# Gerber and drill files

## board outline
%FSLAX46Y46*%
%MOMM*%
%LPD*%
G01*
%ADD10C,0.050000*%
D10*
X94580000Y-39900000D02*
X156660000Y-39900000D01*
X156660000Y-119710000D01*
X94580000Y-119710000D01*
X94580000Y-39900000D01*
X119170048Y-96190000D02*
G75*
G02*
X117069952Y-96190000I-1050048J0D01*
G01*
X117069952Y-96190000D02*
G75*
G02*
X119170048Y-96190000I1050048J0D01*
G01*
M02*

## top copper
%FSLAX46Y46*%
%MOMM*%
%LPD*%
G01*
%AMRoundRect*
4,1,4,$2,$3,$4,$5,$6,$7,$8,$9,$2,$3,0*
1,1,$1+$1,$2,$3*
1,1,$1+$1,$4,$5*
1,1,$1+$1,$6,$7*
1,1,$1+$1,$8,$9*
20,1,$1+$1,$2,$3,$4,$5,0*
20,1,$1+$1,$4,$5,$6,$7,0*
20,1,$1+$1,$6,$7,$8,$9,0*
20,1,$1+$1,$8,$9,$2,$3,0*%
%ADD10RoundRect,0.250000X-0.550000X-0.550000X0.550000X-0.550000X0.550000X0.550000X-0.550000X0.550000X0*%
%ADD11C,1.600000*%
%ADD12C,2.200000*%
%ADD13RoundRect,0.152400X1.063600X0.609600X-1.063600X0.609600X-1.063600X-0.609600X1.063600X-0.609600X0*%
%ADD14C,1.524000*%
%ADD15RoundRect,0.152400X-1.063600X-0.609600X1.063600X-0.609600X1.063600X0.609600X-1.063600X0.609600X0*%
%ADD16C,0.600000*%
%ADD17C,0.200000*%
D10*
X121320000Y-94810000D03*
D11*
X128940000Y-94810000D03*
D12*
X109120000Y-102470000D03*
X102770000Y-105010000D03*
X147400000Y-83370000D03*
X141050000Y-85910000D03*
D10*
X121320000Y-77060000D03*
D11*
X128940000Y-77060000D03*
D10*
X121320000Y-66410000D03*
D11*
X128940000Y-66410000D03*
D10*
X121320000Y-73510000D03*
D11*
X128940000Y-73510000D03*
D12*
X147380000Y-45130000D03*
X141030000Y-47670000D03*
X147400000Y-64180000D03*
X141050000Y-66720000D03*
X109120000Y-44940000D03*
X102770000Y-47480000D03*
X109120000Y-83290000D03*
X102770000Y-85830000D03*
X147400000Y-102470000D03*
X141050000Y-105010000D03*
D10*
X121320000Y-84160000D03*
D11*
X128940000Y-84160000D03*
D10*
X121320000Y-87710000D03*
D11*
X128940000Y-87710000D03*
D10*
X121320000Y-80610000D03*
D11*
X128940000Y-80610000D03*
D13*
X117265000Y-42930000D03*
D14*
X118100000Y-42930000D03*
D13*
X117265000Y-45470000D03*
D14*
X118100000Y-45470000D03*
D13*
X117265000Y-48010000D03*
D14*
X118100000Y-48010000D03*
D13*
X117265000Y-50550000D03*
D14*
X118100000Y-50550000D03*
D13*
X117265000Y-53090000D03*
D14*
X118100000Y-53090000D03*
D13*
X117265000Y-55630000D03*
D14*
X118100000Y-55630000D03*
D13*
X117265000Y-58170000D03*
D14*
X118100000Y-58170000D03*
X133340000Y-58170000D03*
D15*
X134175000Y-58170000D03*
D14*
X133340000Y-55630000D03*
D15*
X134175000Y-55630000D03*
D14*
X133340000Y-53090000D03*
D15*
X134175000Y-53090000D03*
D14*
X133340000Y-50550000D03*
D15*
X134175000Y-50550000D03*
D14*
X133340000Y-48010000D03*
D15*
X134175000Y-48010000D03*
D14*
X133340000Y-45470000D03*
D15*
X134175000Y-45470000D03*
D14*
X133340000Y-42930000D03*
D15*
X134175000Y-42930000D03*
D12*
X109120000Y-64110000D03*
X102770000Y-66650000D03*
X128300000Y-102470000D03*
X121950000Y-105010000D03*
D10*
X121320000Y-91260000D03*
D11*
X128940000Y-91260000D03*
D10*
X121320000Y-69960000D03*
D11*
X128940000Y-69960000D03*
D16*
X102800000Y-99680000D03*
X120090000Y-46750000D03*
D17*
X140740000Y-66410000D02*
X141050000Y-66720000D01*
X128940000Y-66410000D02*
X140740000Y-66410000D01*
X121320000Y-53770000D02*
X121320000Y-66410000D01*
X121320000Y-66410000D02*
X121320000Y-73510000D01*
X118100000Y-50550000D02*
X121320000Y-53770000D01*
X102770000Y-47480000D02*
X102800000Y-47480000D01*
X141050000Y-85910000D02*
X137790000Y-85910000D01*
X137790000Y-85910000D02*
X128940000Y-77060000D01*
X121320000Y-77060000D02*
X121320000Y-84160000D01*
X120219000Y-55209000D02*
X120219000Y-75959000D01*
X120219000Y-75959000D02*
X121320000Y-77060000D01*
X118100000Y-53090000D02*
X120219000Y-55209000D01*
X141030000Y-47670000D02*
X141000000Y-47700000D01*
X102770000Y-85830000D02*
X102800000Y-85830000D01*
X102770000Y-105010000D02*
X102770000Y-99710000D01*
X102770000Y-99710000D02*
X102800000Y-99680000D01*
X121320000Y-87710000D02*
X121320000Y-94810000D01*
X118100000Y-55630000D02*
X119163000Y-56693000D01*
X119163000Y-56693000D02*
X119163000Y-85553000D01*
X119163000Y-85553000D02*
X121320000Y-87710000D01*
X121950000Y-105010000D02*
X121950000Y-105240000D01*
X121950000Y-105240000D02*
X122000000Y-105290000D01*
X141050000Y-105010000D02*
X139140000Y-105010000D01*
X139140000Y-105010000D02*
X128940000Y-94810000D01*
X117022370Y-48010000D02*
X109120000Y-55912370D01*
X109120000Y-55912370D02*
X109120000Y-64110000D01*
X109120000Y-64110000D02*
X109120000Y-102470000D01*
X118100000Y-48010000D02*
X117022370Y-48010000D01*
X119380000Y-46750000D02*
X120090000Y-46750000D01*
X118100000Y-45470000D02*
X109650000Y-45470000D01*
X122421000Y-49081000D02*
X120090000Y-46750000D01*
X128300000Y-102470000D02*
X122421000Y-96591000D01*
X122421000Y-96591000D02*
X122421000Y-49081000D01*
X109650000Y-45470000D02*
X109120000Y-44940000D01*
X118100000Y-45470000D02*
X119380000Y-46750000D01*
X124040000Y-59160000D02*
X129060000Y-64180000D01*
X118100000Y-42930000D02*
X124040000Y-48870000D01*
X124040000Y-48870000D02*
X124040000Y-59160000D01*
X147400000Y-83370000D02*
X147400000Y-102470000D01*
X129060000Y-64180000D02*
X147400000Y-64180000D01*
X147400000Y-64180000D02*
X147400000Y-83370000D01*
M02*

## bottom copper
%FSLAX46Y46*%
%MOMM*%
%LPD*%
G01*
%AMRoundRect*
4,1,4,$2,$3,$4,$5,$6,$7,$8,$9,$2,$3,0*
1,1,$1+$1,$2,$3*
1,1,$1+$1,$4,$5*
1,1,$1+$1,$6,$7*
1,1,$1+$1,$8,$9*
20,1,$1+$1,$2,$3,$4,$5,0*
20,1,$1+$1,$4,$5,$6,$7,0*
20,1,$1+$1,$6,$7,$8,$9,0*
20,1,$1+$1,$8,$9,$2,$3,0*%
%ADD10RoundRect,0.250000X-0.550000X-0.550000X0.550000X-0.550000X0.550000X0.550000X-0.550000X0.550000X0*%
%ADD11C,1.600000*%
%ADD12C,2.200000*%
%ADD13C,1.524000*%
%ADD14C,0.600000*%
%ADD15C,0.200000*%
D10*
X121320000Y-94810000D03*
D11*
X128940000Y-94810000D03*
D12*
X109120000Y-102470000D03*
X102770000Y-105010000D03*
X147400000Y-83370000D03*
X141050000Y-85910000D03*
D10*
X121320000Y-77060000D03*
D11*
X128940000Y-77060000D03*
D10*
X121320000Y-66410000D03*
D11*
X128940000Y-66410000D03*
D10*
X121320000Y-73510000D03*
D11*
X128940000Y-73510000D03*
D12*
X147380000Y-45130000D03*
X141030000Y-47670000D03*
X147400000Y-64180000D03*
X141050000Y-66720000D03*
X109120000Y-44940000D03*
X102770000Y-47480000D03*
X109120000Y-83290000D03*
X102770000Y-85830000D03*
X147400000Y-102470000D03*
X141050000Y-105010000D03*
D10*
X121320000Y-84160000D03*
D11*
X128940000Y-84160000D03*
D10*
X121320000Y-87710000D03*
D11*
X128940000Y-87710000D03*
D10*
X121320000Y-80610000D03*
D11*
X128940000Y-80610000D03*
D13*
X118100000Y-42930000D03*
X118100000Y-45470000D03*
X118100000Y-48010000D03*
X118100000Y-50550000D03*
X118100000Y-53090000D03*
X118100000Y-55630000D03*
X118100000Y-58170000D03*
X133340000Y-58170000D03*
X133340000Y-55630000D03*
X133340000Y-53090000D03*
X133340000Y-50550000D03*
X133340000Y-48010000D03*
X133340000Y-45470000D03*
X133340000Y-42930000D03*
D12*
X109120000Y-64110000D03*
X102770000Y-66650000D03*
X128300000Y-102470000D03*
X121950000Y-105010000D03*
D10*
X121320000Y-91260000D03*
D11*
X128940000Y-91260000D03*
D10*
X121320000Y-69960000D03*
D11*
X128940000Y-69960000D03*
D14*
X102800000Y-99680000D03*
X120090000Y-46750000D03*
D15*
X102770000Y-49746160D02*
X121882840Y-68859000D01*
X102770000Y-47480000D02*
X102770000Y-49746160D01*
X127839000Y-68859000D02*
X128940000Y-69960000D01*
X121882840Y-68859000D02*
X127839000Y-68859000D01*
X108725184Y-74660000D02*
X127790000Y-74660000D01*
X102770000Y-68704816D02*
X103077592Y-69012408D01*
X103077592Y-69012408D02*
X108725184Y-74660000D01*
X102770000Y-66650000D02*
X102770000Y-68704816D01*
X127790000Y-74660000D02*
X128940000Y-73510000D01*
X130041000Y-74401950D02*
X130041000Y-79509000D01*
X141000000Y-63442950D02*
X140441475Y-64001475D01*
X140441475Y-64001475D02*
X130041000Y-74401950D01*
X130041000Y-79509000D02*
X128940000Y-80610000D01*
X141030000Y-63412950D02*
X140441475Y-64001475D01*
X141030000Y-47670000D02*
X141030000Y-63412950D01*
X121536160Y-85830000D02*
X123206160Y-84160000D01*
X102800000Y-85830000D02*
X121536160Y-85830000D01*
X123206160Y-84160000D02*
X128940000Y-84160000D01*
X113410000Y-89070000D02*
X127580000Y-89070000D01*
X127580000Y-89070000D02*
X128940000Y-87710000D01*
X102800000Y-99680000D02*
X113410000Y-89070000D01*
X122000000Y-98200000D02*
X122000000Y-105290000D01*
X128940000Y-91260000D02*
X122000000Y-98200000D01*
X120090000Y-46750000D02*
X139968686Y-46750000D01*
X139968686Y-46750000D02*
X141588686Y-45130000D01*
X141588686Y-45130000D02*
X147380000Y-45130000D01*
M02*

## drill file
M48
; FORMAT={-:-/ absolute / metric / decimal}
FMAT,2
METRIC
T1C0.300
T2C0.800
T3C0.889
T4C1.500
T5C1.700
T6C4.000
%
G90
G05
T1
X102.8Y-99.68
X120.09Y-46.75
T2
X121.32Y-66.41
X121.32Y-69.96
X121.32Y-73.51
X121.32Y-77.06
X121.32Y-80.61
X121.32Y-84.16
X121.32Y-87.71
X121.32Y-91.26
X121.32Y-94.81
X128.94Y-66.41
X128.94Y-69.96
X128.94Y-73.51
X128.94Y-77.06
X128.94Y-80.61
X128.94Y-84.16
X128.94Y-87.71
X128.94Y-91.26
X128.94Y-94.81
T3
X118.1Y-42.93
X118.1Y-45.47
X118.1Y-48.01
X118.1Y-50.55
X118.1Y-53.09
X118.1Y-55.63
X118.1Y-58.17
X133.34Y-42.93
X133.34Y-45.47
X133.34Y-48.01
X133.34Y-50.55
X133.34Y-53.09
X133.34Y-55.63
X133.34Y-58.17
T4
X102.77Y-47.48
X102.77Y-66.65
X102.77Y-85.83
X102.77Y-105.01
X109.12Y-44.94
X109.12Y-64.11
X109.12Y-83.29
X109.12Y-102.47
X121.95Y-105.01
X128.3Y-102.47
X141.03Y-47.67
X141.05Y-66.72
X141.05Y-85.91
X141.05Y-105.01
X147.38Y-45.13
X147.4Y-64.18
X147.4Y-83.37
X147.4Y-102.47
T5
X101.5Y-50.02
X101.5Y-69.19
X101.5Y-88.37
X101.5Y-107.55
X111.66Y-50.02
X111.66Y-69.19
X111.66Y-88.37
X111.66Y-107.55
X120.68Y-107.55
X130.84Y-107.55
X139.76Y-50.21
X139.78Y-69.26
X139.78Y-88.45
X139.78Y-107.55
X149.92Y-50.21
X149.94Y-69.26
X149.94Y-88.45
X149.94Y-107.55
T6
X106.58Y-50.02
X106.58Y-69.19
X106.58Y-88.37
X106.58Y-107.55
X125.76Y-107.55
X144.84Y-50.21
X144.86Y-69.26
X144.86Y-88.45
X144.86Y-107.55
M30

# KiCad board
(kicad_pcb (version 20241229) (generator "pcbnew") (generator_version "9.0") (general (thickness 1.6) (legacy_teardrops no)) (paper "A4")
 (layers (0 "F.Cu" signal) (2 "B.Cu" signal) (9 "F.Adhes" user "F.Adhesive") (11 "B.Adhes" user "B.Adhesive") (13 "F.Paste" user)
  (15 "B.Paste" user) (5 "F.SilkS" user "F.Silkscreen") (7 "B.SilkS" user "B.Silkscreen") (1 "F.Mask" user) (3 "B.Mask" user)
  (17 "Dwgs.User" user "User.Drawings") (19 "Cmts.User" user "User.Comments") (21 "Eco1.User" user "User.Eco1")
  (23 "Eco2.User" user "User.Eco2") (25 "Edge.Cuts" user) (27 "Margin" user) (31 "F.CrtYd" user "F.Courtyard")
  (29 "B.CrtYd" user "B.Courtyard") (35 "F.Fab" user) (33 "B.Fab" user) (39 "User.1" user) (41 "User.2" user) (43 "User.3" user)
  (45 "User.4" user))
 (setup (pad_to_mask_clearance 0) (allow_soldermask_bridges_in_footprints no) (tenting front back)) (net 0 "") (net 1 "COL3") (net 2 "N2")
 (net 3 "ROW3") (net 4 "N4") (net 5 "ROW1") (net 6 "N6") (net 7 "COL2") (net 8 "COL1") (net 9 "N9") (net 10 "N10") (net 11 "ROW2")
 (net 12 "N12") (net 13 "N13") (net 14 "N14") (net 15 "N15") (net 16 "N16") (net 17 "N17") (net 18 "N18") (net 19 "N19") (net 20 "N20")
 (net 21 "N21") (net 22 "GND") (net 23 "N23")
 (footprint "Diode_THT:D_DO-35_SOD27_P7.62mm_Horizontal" (layer "F.Cu") (at 121.32 94.81)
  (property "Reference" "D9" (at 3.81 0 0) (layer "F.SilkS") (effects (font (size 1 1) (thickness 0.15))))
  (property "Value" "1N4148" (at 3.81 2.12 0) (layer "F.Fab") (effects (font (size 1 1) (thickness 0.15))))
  (pad "1" thru_hole roundrect (at 0 0) (size 1.6 1.6) (drill 0.8) (layers "*.Cu" "*.Mask") (remove_unused_layers no)
   (roundrect_rratio 0.15625) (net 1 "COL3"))
  (pad "2" thru_hole circle (at 7.62 0) (size 1.6 1.6) (drill 0.8) (layers "*.Cu" "*.Mask") (remove_unused_layers no) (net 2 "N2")))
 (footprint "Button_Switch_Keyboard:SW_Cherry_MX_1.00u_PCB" (layer "F.Cu") (at 109.12 102.47)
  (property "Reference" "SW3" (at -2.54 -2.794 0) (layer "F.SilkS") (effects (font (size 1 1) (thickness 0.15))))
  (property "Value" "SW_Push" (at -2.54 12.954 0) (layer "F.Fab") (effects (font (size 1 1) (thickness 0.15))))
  (pad "" np_thru_hole circle (at -7.62 5.08) (size 1.7 1.7) (drill 1.7) (layers "*.Cu" "*.Mask"))
  (pad "" np_thru_hole circle (at -2.54 5.08) (size 4 4) (drill 4) (layers "*.Cu" "*.Mask"))
  (pad "" np_thru_hole circle (at 2.54 5.08) (size 1.7 1.7) (drill 1.7) (layers "*.Cu" "*.Mask"))
  (pad "1" thru_hole circle (at 0 0) (size 2.2 2.2) (drill 1.5) (layers "*.Cu" "*.Mask") (remove_unused_layers no) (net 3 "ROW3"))
  (pad "2" thru_hole circle (at -6.35 2.54) (size 2.2 2.2) (drill 1.5) (layers "*.Cu" "*.Mask") (remove_unused_layers no) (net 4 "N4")))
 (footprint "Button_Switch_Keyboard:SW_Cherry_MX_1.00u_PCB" (layer "F.Cu") (at 147.4 83.37)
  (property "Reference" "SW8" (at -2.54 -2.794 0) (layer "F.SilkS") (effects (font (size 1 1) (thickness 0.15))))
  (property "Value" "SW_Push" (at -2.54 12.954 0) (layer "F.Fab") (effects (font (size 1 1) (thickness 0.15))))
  (pad "" np_thru_hole circle (at -7.62 5.08) (size 1.7 1.7) (drill 1.7) (layers "*.Cu" "*.Mask"))
  (pad "" np_thru_hole circle (at -2.54 5.08) (size 4 4) (drill 4) (layers "*.Cu" "*.Mask"))
  (pad "" np_thru_hole circle (at 2.54 5.08) (size 1.7 1.7) (drill 1.7) (layers "*.Cu" "*.Mask"))
  (pad "1" thru_hole circle (at 0 0) (size 2.2 2.2) (drill 1.5) (layers "*.Cu" "*.Mask") (remove_unused_layers no) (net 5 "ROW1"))
  (pad "2" thru_hole circle (at -6.35 2.54) (size 2.2 2.2) (drill 1.5) (layers "*.Cu" "*.Mask") (remove_unused_layers no) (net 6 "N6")))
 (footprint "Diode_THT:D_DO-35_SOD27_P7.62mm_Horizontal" (layer "F.Cu") (at 121.32 77.06)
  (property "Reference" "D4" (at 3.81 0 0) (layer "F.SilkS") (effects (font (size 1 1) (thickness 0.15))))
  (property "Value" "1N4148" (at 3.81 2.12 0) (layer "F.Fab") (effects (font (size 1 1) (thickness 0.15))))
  (pad "1" thru_hole roundrect (at 0 0) (size 1.6 1.6) (drill 0.8) (layers "*.Cu" "*.Mask") (remove_unused_layers no)
   (roundrect_rratio 0.15625) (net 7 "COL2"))
  (pad "2" thru_hole circle (at 7.62 0) (size 1.6 1.6) (drill 0.8) (layers "*.Cu" "*.Mask") (remove_unused_layers no) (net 6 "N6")))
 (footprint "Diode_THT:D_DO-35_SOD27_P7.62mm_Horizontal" (layer "F.Cu") (at 121.32 66.41)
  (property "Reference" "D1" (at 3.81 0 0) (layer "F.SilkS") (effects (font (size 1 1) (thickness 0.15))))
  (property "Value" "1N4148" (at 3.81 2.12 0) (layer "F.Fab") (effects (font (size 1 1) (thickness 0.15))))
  (pad "1" thru_hole roundrect (at 0 0) (size 1.6 1.6) (drill 0.8) (layers "*.Cu" "*.Mask") (remove_unused_layers no)
   (roundrect_rratio 0.15625) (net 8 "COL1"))
  (pad "2" thru_hole circle (at 7.62 0) (size 1.6 1.6) (drill 0.8) (layers "*.Cu" "*.Mask") (remove_unused_layers no) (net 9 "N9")))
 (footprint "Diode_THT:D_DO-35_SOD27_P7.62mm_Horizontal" (layer "F.Cu") (at 121.32 73.51)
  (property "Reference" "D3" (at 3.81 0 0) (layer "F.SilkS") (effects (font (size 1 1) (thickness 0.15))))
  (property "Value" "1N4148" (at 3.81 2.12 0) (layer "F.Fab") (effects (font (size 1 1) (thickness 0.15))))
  (pad "1" thru_hole roundrect (at 0 0) (size 1.6 1.6) (drill 0.8) (layers "*.Cu" "*.Mask") (remove_unused_layers no)
   (roundrect_rratio 0.15625) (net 8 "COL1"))
  (pad "2" thru_hole circle (at 7.62 0) (size 1.6 1.6) (drill 0.8) (layers "*.Cu" "*.Mask") (remove_unused_layers no) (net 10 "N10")))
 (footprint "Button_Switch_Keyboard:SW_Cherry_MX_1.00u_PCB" (layer "F.Cu") (at 147.38 45.13)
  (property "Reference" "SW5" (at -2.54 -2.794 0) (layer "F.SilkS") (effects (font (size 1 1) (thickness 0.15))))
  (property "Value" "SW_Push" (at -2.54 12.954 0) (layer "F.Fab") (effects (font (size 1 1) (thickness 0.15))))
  (pad "" np_thru_hole circle (at -7.62 5.08) (size 1.7 1.7) (drill 1.7) (layers "*.Cu" "*.Mask"))
  (pad "" np_thru_hole circle (at -2.54 5.08) (size 4 4) (drill 4) (layers "*.Cu" "*.Mask"))
  (pad "" np_thru_hole circle (at 2.54 5.08) (size 1.7 1.7) (drill 1.7) (layers "*.Cu" "*.Mask"))
  (pad "1" thru_hole circle (at 0 0) (size 2.2 2.2) (drill 1.5) (layers "*.Cu" "*.Mask") (remove_unused_layers no) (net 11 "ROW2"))
  (pad "2" thru_hole circle (at -6.35 2.54) (size 2.2 2.2) (drill 1.5) (layers "*.Cu" "*.Mask") (remove_unused_layers no) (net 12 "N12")))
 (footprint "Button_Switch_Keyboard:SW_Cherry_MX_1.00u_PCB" (layer "F.Cu") (at 147.4 64.18)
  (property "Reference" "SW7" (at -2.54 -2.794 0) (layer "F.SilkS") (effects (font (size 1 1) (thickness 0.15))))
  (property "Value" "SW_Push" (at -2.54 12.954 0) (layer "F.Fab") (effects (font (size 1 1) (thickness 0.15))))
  (pad "" np_thru_hole circle (at -7.62 5.08) (size 1.7 1.7) (drill 1.7) (layers "*.Cu" "*.Mask"))
  (pad "" np_thru_hole circle (at -2.54 5.08) (size 4 4) (drill 4) (layers "*.Cu" "*.Mask"))
  (pad "" np_thru_hole circle (at 2.54 5.08) (size 1.7 1.7) (drill 1.7) (layers "*.Cu" "*.Mask"))
  (pad "1" thru_hole circle (at 0 0) (size 2.2 2.2) (drill 1.5) (layers "*.Cu" "*.Mask") (remove_unused_layers no) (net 5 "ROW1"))
  (pad "2" thru_hole circle (at -6.35 2.54) (size 2.2 2.2) (drill 1.5) (layers "*.Cu" "*.Mask") (remove_unused_layers no) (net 9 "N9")))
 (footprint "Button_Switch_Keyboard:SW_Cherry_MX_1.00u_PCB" (layer "F.Cu") (at 109.12 44.94)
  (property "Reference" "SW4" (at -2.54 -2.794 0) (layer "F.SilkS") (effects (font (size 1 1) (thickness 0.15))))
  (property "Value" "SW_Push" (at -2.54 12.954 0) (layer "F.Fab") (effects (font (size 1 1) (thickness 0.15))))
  (pad "" np_thru_hole circle (at -7.62 5.08) (size 1.7 1.7) (drill 1.7) (layers "*.Cu" "*.Mask"))
  (pad "" np_thru_hole circle (at -2.54 5.08) (size 4 4) (drill 4) (layers "*.Cu" "*.Mask"))
  (pad "" np_thru_hole circle (at 2.54 5.08) (size 1.7 1.7) (drill 1.7) (layers "*.Cu" "*.Mask"))
  (pad "1" thru_hole circle (at 0 0) (size 2.2 2.2) (drill 1.5) (layers "*.Cu" "*.Mask") (remove_unused_layers no) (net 11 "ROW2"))
  (pad "2" thru_hole circle (at -6.35 2.54) (size 2.2 2.2) (drill 1.5) (layers "*.Cu" "*.Mask") (remove_unused_layers no) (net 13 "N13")))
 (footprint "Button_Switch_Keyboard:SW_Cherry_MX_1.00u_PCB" (layer "F.Cu") (at 109.12 83.29)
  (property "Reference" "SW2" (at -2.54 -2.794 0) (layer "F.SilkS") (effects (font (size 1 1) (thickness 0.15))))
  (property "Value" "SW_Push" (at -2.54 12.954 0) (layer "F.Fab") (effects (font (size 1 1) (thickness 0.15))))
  (pad "" np_thru_hole circle (at -7.62 5.08) (size 1.7 1.7) (drill 1.7) (layers "*.Cu" "*.Mask"))
  (pad "" np_thru_hole circle (at -2.54 5.08) (size 4 4) (drill 4) (layers "*.Cu" "*.Mask"))
  (pad "" np_thru_hole circle (at 2.54 5.08) (size 1.7 1.7) (drill 1.7) (layers "*.Cu" "*.Mask"))
  (pad "1" thru_hole circle (at 0 0) (size 2.2 2.2) (drill 1.5) (layers "*.Cu" "*.Mask") (remove_unused_layers no) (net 3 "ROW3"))
  (pad "2" thru_hole circle (at -6.35 2.54) (size 2.2 2.2) (drill 1.5) (layers "*.Cu" "*.Mask") (remove_unused_layers no) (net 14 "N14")))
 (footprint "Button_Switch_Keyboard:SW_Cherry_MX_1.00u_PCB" (layer "F.Cu") (at 147.4 102.47)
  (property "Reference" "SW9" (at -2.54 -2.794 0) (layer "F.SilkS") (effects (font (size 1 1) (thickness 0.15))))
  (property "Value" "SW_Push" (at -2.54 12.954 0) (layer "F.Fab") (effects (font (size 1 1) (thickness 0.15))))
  (pad "" np_thru_hole circle (at -7.62 5.08) (size 1.7 1.7) (drill 1.7) (layers "*.Cu" "*.Mask"))
  (pad "" np_thru_hole circle (at -2.54 5.08) (size 4 4) (drill 4) (layers "*.Cu" "*.Mask"))
  (pad "" np_thru_hole circle (at 2.54 5.08) (size 1.7 1.7) (drill 1.7) (layers "*.Cu" "*.Mask"))
  (pad "1" thru_hole circle (at 0 0) (size 2.2 2.2) (drill 1.5) (layers "*.Cu" "*.Mask") (remove_unused_layers no) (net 5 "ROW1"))
  (pad "2" thru_hole circle (at -6.35 2.54) (size 2.2 2.2) (drill 1.5) (layers "*.Cu" "*.Mask") (remove_unused_layers no) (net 2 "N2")))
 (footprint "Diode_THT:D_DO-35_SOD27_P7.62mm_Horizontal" (layer "F.Cu") (at 121.32 84.16)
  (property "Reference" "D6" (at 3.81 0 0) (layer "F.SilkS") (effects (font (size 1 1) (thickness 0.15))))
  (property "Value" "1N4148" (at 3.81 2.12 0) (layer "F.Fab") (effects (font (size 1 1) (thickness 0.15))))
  (pad "1" thru_hole roundrect (at 0 0) (size 1.6 1.6) (drill 0.8) (layers "*.Cu" "*.Mask") (remove_unused_layers no)
   (roundrect_rratio 0.15625) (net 7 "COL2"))
  (pad "2" thru_hole circle (at 7.62 0) (size 1.6 1.6) (drill 0.8) (layers "*.Cu" "*.Mask") (remove_unused_layers no) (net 14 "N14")))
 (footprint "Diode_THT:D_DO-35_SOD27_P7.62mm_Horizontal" (layer "F.Cu") (at 121.32 87.71)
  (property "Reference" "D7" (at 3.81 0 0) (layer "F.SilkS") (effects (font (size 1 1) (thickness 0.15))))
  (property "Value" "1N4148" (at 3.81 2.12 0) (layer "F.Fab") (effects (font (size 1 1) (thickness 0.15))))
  (pad "1" thru_hole roundrect (at 0 0) (size 1.6 1.6) (drill 0.8) (layers "*.Cu" "*.Mask") (remove_unused_layers no)
   (roundrect_rratio 0.15625) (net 1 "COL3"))
  (pad "2" thru_hole circle (at 7.62 0) (size 1.6 1.6) (drill 0.8) (layers "*.Cu" "*.Mask") (remove_unused_layers no) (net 4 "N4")))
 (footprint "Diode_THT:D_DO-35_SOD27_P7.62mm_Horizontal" (layer "F.Cu") (at 121.32 80.61)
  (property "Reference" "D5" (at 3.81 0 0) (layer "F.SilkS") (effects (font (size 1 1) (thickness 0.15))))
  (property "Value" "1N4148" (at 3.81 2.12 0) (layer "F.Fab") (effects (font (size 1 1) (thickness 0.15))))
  (pad "1" thru_hole roundrect (at 0 0) (size 1.6 1.6) (drill 0.8) (layers "*.Cu" "*.Mask") (remove_unused_layers no)
   (roundrect_rratio 0.15625) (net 7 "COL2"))
  (pad "2" thru_hole circle (at 7.62 0) (size 1.6 1.6) (drill 0.8) (layers "*.Cu" "*.Mask") (remove_unused_layers no) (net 12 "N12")))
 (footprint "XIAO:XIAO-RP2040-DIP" (layer "F.Cu") (at 125.72 50.55)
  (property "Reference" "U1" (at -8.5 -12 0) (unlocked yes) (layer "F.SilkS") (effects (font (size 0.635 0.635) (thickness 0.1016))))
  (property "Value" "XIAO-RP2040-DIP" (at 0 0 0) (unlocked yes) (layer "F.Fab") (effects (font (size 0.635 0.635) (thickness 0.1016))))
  (pad "1" smd roundrect (at -8.455 -7.62 180) (size 2.432 1.524) (layers "F.Cu" "F.Mask") (roundrect_rratio 0.1) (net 5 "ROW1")
   (thermal_bridge_angle 45))
  (pad "1" thru_hole circle (at -7.62 -7.62 180) (size 1.524 1.524) (drill 0.889) (layers "*.Cu" "*.Mask") (remove_unused_layers no)
   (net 5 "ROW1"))
  (pad "2" smd roundrect (at -8.455 -5.08 180) (size 2.432 1.524) (layers "F.Cu" "F.Mask") (roundrect_rratio 0.1) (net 11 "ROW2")
   (thermal_bridge_angle 45))
  (pad "2" thru_hole circle (at -7.62 -5.08 180) (size 1.524 1.524) (drill 0.889) (layers "*.Cu" "*.Mask") (remove_unused_layers no)
   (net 11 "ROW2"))
  (pad "3" smd roundrect (at -8.455 -2.54 180) (size 2.432 1.524) (layers "F.Cu" "F.Mask") (roundrect_rratio 0.1) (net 3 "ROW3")
   (thermal_bridge_angle 45))
  (pad "3" thru_hole circle (at -7.62 -2.54 180) (size 1.524 1.524) (drill 0.889) (layers "*.Cu" "*.Mask") (remove_unused_layers no)
   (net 3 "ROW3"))
  (pad "4" smd roundrect (at -8.455 0 180) (size 2.432 1.524) (layers "F.Cu" "F.Mask") (roundrect_rratio 0.1) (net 8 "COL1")
   (thermal_bridge_angle 45))
  (pad "4" thru_hole circle (at -7.62 0 180) (size 1.524 1.524) (drill 0.889) (layers "*.Cu" "*.Mask") (remove_unused_layers no)
   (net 8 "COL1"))
  (pad "5" smd roundrect (at -8.455 2.54 180) (size 2.432 1.524) (layers "F.Cu" "F.Mask") (roundrect_rratio 0.1) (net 7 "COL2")
   (thermal_bridge_angle 45))
  (pad "5" thru_hole circle (at -7.62 2.54 180) (size 1.524 1.524) (drill 0.889) (layers "*.Cu" "*.Mask") (remove_unused_layers no)
   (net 7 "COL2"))
  (pad "6" smd roundrect (at -8.455 5.08 180) (size 2.432 1.524) (layers "F.Cu" "F.Mask") (roundrect_rratio 0.1) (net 1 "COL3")
   (thermal_bridge_angle 45))
  (pad "6" thru_hole circle (at -7.62 5.08 180) (size 1.524 1.524) (drill 0.889) (layers "*.Cu" "*.Mask") (remove_unused_layers no)
   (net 1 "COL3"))
  (pad "7" smd roundrect (at -8.455 7.62 180) (size 2.432 1.524) (layers "F.Cu" "F.Mask") (roundrect_rratio 0.1) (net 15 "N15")
   (thermal_bridge_angle 45))
  (pad "7" thru_hole circle (at -7.62 7.62 180) (size 1.524 1.524) (drill 0.889) (layers "*.Cu" "*.Mask") (remove_unused_layers no)
   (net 15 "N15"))
  (pad "8" thru_hole circle (at 7.62 7.62) (size 1.524 1.524) (drill 0.889) (layers "*.Cu" "*.Mask") (remove_unused_layers no)
   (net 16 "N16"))
  (pad "8" smd roundrect (at 8.455 7.62) (size 2.432 1.524) (layers "F.Cu" "F.Mask") (roundrect_rratio 0.1) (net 16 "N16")
   (thermal_bridge_angle 45))
  (pad "9" thru_hole circle (at 7.62 5.08) (size 1.524 1.524) (drill 0.889) (layers "*.Cu" "*.Mask") (remove_unused_layers no)
   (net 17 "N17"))
  (pad "9" smd roundrect (at 8.455 5.08) (size 2.432 1.524) (layers "F.Cu" "F.Mask") (roundrect_rratio 0.1) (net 17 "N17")
   (thermal_bridge_angle 45))
  (pad "10" thru_hole circle (at 7.62 2.54) (size 1.524 1.524) (drill 0.889) (layers "*.Cu" "*.Mask") (remove_unused_layers no)
   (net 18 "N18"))
  (pad "10" smd roundrect (at 8.455 2.54) (size 2.432 1.524) (layers "F.Cu" "F.Mask") (roundrect_rratio 0.1) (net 18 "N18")
   (thermal_bridge_angle 45))
  (pad "11" thru_hole circle (at 7.62 0) (size 1.524 1.524) (drill 0.889) (layers "*.Cu" "*.Mask") (remove_unused_layers no) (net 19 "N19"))
  (pad "11" smd roundrect (at 8.455 0) (size 2.432 1.524) (layers "F.Cu" "F.Mask") (roundrect_rratio 0.1) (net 19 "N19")
   (thermal_bridge_angle 45))
  (pad "12" thru_hole circle (at 7.62 -2.54) (size 1.524 1.524) (drill 0.889) (layers "*.Cu" "*.Mask") (remove_unused_layers no)
   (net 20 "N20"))
  (pad "12" smd roundrect (at 8.455 -2.54) (size 2.432 1.524) (layers "F.Cu" "F.Mask") (roundrect_rratio 0.1) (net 20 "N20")
   (thermal_bridge_angle 45))
  (pad "13" thru_hole circle (at 7.62 -5.08) (size 1.524 1.524) (drill 0.889) (layers "*.Cu" "*.Mask") (remove_unused_layers no)
   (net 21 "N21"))
  (pad "13" smd roundrect (at 8.455 -5.08) (size 2.432 1.524) (layers "F.Cu" "F.Mask") (roundrect_rratio 0.1) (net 21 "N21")
   (thermal_bridge_angle 45))
  (pad "14" thru_hole circle (at 7.62 -7.62) (size 1.524 1.524) (drill 0.889) (layers "*.Cu" "*.Mask") (remove_unused_layers no)
   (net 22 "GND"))
  (pad "14" smd roundrect (at 8.455 -7.62) (size 2.432 1.524) (layers "F.Cu" "F.Mask") (roundrect_rratio 0.1) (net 22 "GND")
   (thermal_bridge_angle 45)))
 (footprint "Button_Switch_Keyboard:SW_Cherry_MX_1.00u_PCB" (layer "F.Cu") (at 109.12 64.11)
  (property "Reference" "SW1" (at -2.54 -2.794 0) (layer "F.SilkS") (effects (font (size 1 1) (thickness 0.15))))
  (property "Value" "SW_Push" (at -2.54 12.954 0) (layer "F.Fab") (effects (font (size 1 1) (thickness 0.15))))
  (pad "" np_thru_hole circle (at -7.62 5.08) (size 1.7 1.7) (drill 1.7) (layers "*.Cu" "*.Mask"))
  (pad "" np_thru_hole circle (at -2.54 5.08) (size 4 4) (drill 4) (layers "*.Cu" "*.Mask"))
  (pad "" np_thru_hole circle (at 2.54 5.08) (size 1.7 1.7) (drill 1.7) (layers "*.Cu" "*.Mask"))
  (pad "1" thru_hole circle (at 0 0) (size 2.2 2.2) (drill 1.5) (layers "*.Cu" "*.Mask") (remove_unused_layers no) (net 3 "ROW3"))
  (pad "2" thru_hole circle (at -6.35 2.54) (size 2.2 2.2) (drill 1.5) (layers "*.Cu" "*.Mask") (remove_unused_layers no) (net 10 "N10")))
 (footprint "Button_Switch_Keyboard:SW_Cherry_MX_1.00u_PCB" (layer "F.Cu") (at 128.3 102.47)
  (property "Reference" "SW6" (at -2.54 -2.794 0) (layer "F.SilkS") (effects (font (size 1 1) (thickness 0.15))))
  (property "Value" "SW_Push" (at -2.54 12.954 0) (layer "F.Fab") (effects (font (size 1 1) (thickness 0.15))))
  (pad "" np_thru_hole circle (at -7.62 5.08) (size 1.7 1.7) (drill 1.7) (layers "*.Cu" "*.Mask"))
  (pad "" np_thru_hole circle (at -2.54 5.08) (size 4 4) (drill 4) (layers "*.Cu" "*.Mask"))
  (pad "" np_thru_hole circle (at 2.54 5.08) (size 1.7 1.7) (drill 1.7) (layers "*.Cu" "*.Mask"))
  (pad "1" thru_hole circle (at 0 0) (size 2.2 2.2) (drill 1.5) (layers "*.Cu" "*.Mask") (remove_unused_layers no) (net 11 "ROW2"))
  (pad "2" thru_hole circle (at -6.35 2.54) (size 2.2 2.2) (drill 1.5) (layers "*.Cu" "*.Mask") (remove_unused_layers no) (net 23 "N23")))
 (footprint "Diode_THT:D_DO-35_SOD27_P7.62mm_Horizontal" (layer "F.Cu") (at 121.32 91.26)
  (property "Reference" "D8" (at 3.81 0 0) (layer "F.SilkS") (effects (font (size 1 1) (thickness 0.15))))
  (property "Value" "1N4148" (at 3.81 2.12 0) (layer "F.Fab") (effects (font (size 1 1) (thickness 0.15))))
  (pad "1" thru_hole roundrect (at 0 0) (size 1.6 1.6) (drill 0.8) (layers "*.Cu" "*.Mask") (remove_unused_layers no)
   (roundrect_rratio 0.15625) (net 1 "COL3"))
  (pad "2" thru_hole circle (at 7.62 0) (size 1.6 1.6) (drill 0.8) (layers "*.Cu" "*.Mask") (remove_unused_layers no) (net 23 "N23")))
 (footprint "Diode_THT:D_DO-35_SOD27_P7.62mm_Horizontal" (layer "F.Cu") (at 121.32 69.96)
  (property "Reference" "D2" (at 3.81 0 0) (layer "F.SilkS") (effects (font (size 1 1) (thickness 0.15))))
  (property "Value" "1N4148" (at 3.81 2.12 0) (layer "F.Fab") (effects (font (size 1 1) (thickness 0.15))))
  (pad "1" thru_hole roundrect (at 0 0) (size 1.6 1.6) (drill 0.8) (layers "*.Cu" "*.Mask") (remove_unused_layers no)
   (roundrect_rratio 0.15625) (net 8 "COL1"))
  (pad "2" thru_hole circle (at 7.62 0) (size 1.6 1.6) (drill 0.8) (layers "*.Cu" "*.Mask") (remove_unused_layers no) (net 13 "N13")))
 (gr_rect (start 94.58 39.9) (end 156.66 119.71) (stroke (width 0.05) (type default)) (fill no) (layer "Edge.Cuts"))
 (gr_circle (center 118.12 96.19) (end 117.07 96.18) (stroke (width 0.05) (type default)) (fill no) (layer "Edge.Cuts"))
 (segment (start 140.74 66.41) (end 141.05 66.72) (width 0.2) (layer "F.Cu") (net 9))
 (segment (start 128.94 66.41) (end 140.74 66.41) (width 0.2) (layer "F.Cu") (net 9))
 (segment (start 121.32 53.77) (end 121.32 66.41) (width 0.2) (layer "F.Cu") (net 8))
 (segment (start 121.32 66.41) (end 121.32 73.51) (width 0.2) (layer "F.Cu") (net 8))
 (segment (start 118.1 50.55) (end 121.32 53.77) (width 0.2) (layer "F.Cu") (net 8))
 (segment (start 102.77 47.48) (end 102.8 47.48) (width 0.2) (layer "F.Cu") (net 13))
 (segment (start 102.77 49.74616) (end 121.88284 68.859) (width 0.2) (layer "B.Cu") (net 13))
 (segment (start 102.77 47.48) (end 102.77 49.74616) (width 0.2) (layer "B.Cu") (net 13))
 (segment (start 127.839 68.859) (end 128.94 69.96) (width 0.2) (layer "B.Cu") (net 13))
 (segment (start 121.88284 68.859) (end 127.839 68.859) (width 0.2) (layer "B.Cu") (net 13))
 (segment (start 108.725184 74.66) (end 127.79 74.66) (width 0.2) (layer "B.Cu") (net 10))
 (segment (start 102.77 68.704816) (end 103.077592 69.012408) (width 0.2) (layer "B.Cu") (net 10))
 (segment (start 103.077592 69.012408) (end 108.725184 74.66) (width 0.2) (layer "B.Cu") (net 10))
 (segment (start 102.77 66.65) (end 102.77 68.704816) (width 0.2) (layer "B.Cu") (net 10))
 (segment (start 127.79 74.66) (end 128.94 73.51) (width 0.2) (layer "B.Cu") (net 10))
 (segment (start 141.05 85.91) (end 137.79 85.91) (width 0.2) (layer "F.Cu") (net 6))
 (segment (start 137.79 85.91) (end 128.94 77.06) (width 0.2) (layer "F.Cu") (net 6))
 (segment (start 121.32 77.06) (end 121.32 84.16) (width 0.2) (layer "F.Cu") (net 7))
 (segment (start 120.219 55.209) (end 120.219 75.959) (width 0.2) (layer "F.Cu") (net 7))
 (segment (start 120.219 75.959) (end 121.32 77.06) (width 0.2) (layer "F.Cu") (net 7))
 (segment (start 118.1 53.09) (end 120.219 55.209) (width 0.2) (layer "F.Cu") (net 7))
 (segment (start 141.03 47.67) (end 141 47.7) (width 0.2) (layer "F.Cu") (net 12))
 (segment (start 130.041 74.40195) (end 130.041 79.509) (width 0.2) (layer "B.Cu") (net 12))
 (segment (start 141 63.44295) (end 140.441475 64.001475) (width 0.2) (layer "B.Cu") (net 12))
 (segment (start 140.441475 64.001475) (end 130.041 74.40195) (width 0.2) (layer "B.Cu") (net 12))
 (segment (start 130.041 79.509) (end 128.94 80.61) (width 0.2) (layer "B.Cu") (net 12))
 (segment (start 141.03 63.41295) (end 140.441475 64.001475) (width 0.2) (layer "B.Cu") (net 12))
 (segment (start 141.03 47.67) (end 141.03 63.41295) (width 0.2) (layer "B.Cu") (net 12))
 (segment (start 102.77 85.83) (end 102.8 85.83) (width 0.2) (layer "F.Cu") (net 14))
 (segment (start 121.53616 85.83) (end 123.20616 84.16) (width 0.2) (layer "B.Cu") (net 14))
 (segment (start 102.8 85.83) (end 121.53616 85.83) (width 0.2) (layer "B.Cu") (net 14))
 (segment (start 123.20616 84.16) (end 128.94 84.16) (width 0.2) (layer "B.Cu") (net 14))
 (segment (start 102.77 105.01) (end 102.77 99.71) (width 0.2) (layer "F.Cu") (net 4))
 (segment (start 102.77 99.71) (end 102.8 99.68) (width 0.2) (layer "F.Cu") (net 4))
 (via (at 102.8 99.68) (size 0.6) (drill 0.3) (layers "F.Cu" "B.Cu") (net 4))
 (segment (start 113.41 89.07) (end 127.58 89.07) (width 0.2) (layer "B.Cu") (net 4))
 (segment (start 127.58 89.07) (end 128.94 87.71) (width 0.2) (layer "B.Cu") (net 4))
 (segment (start 102.8 99.68) (end 113.41 89.07) (width 0.2) (layer "B.Cu") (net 4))
 (segment (start 121.32 87.71) (end 121.32 94.81) (width 0.2) (layer "F.Cu") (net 1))
 (segment (start 118.1 55.63) (end 119.163 56.693) (width 0.2) (layer "F.Cu") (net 1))
 (segment (start 119.163 56.693) (end 119.163 85.553) (width 0.2) (layer "F.Cu") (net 1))
 (segment (start 119.163 85.553) (end 121.32 87.71) (width 0.2) (layer "F.Cu") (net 1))
 (segment (start 121.95 105.01) (end 121.95 105.24) (width 0.2) (layer "F.Cu") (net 23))
 (segment (start 121.95 105.24) (end 122 105.29) (width 0.2) (layer "F.Cu") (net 23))
 (segment (start 122 98.2) (end 122 105.29) (width 0.2) (layer "B.Cu") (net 23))
 (segment (start 128.94 91.26) (end 122 98.2) (width 0.2) (layer "B.Cu") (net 23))
 (segment (start 141.05 105.01) (end 139.14 105.01) (width 0.2) (layer "F.Cu") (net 2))
 (segment (start 139.14 105.01) (end 128.94 94.81) (width 0.2) (layer "F.Cu") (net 2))
 (segment (start 117.02237 48.01) (end 109.12 55.91237) (width 0.2) (layer "F.Cu") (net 3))
 (segment (start 109.12 55.91237) (end 109.12 64.11) (width 0.2) (layer "F.Cu") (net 3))
 (segment (start 109.12 64.11) (end 109.12 102.47) (width 0.2) (layer "F.Cu") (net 3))
 (segment (start 118.1 48.01) (end 117.02237 48.01) (width 0.2) (layer "F.Cu") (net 3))
 (segment (start 119.38 46.75) (end 120.09 46.75) (width 0.2) (layer "F.Cu") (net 11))
 (segment (start 118.1 45.47) (end 109.65 45.47) (width 0.2) (layer "F.Cu") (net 11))
 (segment (start 122.421 49.081) (end 120.09 46.75) (width 0.2) (layer "F.Cu") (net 11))
 (segment (start 128.3 102.47) (end 122.421 96.591) (width 0.2) (layer "F.Cu") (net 11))
 (segment (start 122.421 96.591) (end 122.421 49.081) (width 0.2) (layer "F.Cu") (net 11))
 (segment (start 109.65 45.47) (end 109.12 44.94) (width 0.2) (layer "F.Cu") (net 11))
 (segment (start 118.1 45.47) (end 119.38 46.75) (width 0.2) (layer "F.Cu") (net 11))
 (via (at 120.09 46.75) (size 0.6) (drill 0.3) (layers "F.Cu" "B.Cu") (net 11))
 (segment (start 120.09 46.75) (end 139.968686 46.75) (width 0.2) (layer "B.Cu") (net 11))
 (segment (start 139.968686 46.75) (end 141.588686 45.13) (width 0.2) (layer "B.Cu") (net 11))
 (segment (start 141.588686 45.13) (end 147.38 45.13) (width 0.2) (layer "B.Cu") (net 11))
 (segment (start 124.04 59.16) (end 129.06 64.18) (width 0.2) (layer "F.Cu") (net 5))
 (segment (start 118.1 42.93) (end 124.04 48.87) (width 0.2) (layer "F.Cu") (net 5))
 (segment (start 124.04 48.87) (end 124.04 59.16) (width 0.2) (layer "F.Cu") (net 5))
 (segment (start 147.4 83.37) (end 147.4 102.47) (width 0.2) (layer "F.Cu") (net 5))
 (segment (start 129.06 64.18) (end 147.4 64.18) (width 0.2) (layer "F.Cu") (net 5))
 (segment (start 147.4 64.18) (end 147.4 83.37) (width 0.2) (layer "F.Cu") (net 5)))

